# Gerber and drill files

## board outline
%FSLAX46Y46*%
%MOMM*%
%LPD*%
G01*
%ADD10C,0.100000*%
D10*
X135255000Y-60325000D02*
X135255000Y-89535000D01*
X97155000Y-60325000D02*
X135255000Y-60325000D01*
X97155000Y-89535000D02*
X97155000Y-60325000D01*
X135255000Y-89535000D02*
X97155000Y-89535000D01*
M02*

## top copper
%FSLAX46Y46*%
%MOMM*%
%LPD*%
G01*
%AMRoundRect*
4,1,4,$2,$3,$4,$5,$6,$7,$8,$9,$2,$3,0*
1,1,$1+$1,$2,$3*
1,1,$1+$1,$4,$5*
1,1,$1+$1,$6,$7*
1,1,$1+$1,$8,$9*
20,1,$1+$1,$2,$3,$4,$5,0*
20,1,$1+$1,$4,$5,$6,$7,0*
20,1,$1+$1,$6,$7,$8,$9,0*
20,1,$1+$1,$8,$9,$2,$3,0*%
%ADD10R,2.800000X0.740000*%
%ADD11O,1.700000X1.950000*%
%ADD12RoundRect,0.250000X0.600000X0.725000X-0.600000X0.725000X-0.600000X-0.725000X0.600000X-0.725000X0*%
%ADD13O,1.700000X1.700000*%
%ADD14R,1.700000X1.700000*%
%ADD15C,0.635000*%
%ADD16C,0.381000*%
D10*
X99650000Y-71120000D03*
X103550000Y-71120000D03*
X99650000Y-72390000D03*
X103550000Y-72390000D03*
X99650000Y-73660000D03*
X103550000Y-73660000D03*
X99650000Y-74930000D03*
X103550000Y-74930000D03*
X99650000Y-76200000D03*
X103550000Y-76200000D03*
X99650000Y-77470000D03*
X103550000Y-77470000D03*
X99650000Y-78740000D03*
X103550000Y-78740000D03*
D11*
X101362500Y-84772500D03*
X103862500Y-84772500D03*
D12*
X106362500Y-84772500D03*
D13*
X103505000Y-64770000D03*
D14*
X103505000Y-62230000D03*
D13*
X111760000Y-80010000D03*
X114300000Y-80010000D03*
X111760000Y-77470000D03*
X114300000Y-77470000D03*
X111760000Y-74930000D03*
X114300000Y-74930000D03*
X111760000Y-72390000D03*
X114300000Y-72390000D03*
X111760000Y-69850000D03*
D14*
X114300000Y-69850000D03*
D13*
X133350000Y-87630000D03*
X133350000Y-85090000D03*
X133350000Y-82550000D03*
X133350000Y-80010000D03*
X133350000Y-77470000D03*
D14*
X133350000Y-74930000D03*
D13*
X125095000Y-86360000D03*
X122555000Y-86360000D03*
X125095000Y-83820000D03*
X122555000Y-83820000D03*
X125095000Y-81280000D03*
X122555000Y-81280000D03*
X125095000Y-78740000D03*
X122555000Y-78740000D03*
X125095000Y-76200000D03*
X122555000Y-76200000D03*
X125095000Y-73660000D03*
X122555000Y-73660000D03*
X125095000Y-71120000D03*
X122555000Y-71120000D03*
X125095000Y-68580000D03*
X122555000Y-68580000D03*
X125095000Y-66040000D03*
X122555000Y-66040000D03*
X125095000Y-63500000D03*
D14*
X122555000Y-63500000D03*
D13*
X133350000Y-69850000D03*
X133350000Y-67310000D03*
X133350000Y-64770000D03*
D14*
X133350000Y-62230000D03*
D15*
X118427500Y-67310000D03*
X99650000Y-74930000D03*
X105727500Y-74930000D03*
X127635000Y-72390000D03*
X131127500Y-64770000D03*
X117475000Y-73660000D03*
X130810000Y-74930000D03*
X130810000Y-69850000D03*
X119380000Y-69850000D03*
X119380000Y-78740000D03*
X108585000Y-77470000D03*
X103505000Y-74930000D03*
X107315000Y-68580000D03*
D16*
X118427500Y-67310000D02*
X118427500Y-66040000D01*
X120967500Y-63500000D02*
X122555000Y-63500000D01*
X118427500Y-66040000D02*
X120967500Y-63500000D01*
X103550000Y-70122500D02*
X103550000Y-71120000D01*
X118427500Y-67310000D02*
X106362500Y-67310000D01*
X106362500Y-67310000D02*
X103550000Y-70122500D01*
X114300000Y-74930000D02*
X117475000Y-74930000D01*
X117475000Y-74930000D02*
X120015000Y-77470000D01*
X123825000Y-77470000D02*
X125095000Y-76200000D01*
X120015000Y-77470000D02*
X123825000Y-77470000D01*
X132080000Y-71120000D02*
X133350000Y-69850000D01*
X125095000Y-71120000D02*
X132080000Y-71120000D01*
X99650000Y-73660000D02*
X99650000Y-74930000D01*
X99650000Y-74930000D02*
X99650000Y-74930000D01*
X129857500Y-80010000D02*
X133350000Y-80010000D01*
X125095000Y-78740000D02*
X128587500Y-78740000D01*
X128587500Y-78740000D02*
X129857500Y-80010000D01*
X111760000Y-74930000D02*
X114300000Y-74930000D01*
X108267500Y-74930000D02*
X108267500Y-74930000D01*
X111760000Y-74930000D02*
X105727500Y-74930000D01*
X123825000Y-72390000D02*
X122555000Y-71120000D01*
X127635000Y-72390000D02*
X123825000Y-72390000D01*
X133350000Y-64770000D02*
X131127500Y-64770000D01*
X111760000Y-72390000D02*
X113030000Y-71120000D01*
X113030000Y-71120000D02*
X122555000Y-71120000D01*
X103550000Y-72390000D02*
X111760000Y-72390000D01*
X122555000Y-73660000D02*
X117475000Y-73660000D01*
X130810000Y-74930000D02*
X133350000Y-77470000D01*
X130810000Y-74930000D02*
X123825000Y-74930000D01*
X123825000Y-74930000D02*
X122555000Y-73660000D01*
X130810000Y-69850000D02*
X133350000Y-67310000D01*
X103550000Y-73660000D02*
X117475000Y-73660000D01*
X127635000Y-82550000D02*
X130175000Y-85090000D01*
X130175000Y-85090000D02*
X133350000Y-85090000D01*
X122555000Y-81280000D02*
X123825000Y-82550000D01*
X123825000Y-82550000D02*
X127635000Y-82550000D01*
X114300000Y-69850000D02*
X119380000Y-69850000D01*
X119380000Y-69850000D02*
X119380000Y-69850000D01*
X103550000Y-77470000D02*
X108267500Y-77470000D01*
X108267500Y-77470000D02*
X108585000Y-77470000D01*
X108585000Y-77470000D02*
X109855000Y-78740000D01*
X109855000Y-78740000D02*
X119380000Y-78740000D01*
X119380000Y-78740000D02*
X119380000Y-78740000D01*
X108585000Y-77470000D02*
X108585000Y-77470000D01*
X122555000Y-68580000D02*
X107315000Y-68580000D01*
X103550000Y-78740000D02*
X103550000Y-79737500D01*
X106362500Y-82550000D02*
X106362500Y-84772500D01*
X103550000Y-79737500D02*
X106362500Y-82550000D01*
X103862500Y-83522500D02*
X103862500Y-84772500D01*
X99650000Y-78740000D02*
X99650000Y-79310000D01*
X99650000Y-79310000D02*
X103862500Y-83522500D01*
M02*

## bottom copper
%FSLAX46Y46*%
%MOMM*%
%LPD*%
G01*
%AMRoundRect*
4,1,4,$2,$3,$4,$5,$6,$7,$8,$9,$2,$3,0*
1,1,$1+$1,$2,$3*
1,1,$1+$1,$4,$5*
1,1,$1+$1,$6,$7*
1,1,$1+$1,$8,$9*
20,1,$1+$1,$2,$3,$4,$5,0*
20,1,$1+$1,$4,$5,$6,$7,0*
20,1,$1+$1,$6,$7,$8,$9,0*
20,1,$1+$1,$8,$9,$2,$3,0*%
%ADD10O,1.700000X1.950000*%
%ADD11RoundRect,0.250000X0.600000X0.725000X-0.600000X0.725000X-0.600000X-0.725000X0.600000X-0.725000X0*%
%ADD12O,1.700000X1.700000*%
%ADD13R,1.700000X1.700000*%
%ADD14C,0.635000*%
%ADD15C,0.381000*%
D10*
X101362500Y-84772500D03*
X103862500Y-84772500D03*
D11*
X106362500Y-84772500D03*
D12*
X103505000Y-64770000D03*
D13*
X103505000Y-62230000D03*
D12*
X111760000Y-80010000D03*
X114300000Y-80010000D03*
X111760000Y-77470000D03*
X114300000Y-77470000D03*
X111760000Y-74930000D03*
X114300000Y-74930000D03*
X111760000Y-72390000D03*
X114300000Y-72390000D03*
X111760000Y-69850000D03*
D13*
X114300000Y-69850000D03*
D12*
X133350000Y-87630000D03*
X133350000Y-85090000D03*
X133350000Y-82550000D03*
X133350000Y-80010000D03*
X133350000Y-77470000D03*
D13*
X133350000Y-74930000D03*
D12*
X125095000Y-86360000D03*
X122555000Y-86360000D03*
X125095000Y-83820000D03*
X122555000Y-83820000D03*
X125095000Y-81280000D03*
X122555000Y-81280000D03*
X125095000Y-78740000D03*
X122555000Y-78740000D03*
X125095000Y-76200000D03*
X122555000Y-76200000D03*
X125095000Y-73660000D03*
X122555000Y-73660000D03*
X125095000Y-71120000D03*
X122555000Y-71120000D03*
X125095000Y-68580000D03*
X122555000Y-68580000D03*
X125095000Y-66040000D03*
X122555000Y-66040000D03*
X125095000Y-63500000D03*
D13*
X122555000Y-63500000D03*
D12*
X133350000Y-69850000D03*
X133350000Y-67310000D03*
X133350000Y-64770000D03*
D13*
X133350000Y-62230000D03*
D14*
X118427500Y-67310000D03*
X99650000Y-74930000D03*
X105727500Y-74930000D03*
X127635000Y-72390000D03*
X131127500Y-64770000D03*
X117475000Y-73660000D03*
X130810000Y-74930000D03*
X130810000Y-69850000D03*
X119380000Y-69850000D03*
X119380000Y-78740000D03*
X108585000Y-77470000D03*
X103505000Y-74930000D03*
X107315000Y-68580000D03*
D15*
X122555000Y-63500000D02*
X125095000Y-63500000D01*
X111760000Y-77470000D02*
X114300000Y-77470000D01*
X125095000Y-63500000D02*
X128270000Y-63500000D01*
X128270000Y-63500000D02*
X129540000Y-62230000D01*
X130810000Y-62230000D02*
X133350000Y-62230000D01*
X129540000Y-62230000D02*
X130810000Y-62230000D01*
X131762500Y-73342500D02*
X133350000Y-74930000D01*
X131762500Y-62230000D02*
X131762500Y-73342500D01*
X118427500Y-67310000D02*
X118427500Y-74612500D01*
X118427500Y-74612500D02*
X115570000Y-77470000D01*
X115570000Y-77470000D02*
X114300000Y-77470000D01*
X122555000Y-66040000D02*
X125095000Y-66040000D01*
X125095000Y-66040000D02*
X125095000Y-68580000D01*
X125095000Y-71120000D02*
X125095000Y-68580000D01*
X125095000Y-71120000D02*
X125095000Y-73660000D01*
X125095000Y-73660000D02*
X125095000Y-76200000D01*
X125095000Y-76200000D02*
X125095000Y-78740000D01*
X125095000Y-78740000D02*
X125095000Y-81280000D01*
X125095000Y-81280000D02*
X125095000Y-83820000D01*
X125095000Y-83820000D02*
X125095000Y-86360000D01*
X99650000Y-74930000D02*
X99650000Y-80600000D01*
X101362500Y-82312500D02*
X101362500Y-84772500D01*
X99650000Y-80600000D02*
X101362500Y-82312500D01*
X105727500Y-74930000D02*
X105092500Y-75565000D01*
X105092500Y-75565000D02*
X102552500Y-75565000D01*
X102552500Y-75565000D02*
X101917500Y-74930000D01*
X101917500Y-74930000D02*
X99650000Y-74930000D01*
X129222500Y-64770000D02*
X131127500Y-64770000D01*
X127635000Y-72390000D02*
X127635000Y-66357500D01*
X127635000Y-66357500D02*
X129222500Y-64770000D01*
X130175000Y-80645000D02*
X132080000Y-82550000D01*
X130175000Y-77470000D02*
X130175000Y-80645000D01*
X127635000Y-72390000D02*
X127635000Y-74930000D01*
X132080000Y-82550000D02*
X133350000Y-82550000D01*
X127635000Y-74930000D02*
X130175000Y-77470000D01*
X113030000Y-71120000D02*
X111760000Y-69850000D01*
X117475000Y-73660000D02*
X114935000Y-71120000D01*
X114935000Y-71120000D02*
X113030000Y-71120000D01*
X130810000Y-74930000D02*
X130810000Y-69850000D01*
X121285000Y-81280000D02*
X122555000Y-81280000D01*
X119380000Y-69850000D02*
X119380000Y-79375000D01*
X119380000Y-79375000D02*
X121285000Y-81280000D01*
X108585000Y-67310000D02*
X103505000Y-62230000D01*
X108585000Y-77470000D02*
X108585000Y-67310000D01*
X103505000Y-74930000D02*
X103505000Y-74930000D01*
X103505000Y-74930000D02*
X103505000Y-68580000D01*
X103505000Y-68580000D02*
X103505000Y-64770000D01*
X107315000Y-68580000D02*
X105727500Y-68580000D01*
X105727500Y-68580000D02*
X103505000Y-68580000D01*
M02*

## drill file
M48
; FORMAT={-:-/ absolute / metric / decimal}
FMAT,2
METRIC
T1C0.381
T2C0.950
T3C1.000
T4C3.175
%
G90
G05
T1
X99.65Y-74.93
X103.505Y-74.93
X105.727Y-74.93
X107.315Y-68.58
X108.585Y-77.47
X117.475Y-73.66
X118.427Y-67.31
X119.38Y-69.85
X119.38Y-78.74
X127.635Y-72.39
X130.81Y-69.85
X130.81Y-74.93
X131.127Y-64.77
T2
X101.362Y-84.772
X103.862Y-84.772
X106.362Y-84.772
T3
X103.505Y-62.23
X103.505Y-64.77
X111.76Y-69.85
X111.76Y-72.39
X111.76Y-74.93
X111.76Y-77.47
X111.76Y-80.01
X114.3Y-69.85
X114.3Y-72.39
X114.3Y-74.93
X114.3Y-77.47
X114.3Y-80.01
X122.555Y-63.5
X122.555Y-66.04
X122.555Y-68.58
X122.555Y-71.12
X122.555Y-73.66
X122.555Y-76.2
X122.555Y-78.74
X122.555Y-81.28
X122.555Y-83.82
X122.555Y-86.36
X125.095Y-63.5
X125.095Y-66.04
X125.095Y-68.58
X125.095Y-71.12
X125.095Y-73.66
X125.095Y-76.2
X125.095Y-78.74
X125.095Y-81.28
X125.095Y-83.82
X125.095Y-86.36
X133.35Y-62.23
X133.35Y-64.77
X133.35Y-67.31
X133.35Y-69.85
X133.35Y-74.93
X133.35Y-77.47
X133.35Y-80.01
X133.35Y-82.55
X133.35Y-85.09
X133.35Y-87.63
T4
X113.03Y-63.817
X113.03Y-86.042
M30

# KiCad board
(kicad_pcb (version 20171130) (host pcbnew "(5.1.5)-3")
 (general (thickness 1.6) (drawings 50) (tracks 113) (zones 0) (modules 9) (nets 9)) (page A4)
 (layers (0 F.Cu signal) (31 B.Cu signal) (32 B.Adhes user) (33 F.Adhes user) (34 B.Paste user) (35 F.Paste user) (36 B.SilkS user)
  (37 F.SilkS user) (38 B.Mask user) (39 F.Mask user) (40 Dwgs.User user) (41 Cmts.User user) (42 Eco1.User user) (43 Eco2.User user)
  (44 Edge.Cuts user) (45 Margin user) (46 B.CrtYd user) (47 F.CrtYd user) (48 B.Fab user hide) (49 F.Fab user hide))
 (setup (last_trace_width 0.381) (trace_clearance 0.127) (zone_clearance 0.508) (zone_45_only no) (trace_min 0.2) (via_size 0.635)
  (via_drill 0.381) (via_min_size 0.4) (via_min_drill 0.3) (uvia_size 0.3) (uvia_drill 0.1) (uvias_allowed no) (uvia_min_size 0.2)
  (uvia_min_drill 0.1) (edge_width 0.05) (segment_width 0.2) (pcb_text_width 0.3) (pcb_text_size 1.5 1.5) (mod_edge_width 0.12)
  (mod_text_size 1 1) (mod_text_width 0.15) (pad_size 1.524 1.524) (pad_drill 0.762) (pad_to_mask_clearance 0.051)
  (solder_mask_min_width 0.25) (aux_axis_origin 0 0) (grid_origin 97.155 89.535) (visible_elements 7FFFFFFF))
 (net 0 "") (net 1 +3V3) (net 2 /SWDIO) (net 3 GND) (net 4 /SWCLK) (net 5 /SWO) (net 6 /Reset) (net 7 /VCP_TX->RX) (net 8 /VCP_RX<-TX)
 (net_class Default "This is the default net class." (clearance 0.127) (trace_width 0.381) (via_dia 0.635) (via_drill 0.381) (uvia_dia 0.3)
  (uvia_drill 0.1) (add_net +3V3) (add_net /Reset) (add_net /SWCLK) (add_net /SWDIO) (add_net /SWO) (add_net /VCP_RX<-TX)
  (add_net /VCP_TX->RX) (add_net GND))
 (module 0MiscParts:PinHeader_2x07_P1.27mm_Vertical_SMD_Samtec (layer F.Cu) (at 101.6 74.93)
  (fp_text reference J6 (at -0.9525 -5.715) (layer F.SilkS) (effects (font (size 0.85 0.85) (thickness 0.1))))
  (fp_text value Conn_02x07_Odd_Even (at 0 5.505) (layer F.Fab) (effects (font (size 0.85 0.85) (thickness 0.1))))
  (pad 1 smd rect (at -1.95 -3.81) (size 2.8 0.74) (layers F.Cu F.Paste F.Mask))
  (pad 2 smd rect (at 1.95 -3.81) (size 2.8 0.74) (layers F.Cu F.Paste F.Mask) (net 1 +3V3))
  (pad 3 smd rect (at -1.95 -2.54) (size 2.8 0.74) (layers F.Cu F.Paste F.Mask))
  (pad 4 smd rect (at 1.95 -2.54) (size 2.8 0.74) (layers F.Cu F.Paste F.Mask) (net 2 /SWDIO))
  (pad 5 smd rect (at -1.95 -1.27) (size 2.8 0.74) (layers F.Cu F.Paste F.Mask) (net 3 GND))
  (pad 6 smd rect (at 1.95 -1.27) (size 2.8 0.74) (layers F.Cu F.Paste F.Mask) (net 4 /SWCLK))
  (pad 7 smd rect (at -1.95 0) (size 2.8 0.74) (layers F.Cu F.Paste F.Mask) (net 3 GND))
  (pad 8 smd rect (at 1.95 0) (size 2.8 0.74) (layers F.Cu F.Paste F.Mask) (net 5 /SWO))
  (pad 9 smd rect (at -1.95 1.27) (size 2.8 0.74) (layers F.Cu F.Paste F.Mask))
  (pad 10 smd rect (at 1.95 1.27) (size 2.8 0.74) (layers F.Cu F.Paste F.Mask))
  (pad 11 smd rect (at -1.95 2.54) (size 2.8 0.74) (layers F.Cu F.Paste F.Mask))
  (pad 12 smd rect (at 1.95 2.54) (size 2.8 0.74) (layers F.Cu F.Paste F.Mask) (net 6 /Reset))
  (pad 13 smd rect (at -1.95 3.81) (size 2.8 0.74) (layers F.Cu F.Paste F.Mask) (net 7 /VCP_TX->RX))
  (pad 14 smd rect (at 1.95 3.81) (size 2.8 0.74) (layers F.Cu F.Paste F.Mask) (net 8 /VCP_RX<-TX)))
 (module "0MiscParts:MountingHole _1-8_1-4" (layer F.Cu) (at 113.03 63.8175)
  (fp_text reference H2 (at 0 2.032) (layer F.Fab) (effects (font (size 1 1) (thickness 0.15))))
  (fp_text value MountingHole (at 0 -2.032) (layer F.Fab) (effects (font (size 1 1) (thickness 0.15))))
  (pad "" np_thru_hole circle (at 0 0) (size 3.175 3.175) (drill 3.175) (layers *.Cu *.Mask)))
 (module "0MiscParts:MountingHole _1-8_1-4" (layer F.Cu) (at 113.03 86.0425)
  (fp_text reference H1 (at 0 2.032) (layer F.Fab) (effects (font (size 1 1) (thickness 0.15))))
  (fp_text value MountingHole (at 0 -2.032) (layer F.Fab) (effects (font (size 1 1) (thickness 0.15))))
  (pad "" np_thru_hole circle (at 0 0) (size 3.175 3.175) (drill 3.175) (layers *.Cu *.Mask)))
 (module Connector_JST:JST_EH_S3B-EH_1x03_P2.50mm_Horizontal (layer F.Cu) (at 106.3625 84.7725 180)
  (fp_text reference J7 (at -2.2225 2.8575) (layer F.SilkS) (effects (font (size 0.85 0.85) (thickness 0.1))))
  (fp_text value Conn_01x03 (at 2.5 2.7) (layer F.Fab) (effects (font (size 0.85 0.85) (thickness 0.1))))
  (pad 3 thru_hole oval (at 5 0 180) (size 1.7 1.95) (drill 0.95) (layers *.Cu *.Mask) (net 3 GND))
  (pad 2 thru_hole oval (at 2.5 0 180) (size 1.7 1.95) (drill 0.95) (layers *.Cu *.Mask) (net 7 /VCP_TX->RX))
  (pad 1 thru_hole roundrect (at 0 0 180) (size 1.7 1.95) (drill 0.95) (layers *.Cu *.Mask) (roundrect_rratio 0.147059) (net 8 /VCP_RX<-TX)))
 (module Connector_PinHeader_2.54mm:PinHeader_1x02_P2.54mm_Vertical (layer F.Cu) (at 103.505 62.23)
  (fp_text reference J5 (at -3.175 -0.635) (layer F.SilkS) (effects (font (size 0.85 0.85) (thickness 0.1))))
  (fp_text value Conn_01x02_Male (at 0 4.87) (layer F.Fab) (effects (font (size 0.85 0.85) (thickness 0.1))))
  (pad 2 thru_hole oval (at 0 2.54) (size 1.7 1.7) (drill 1) (layers *.Cu *.Mask) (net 5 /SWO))
  (pad 1 thru_hole rect (at 0 0) (size 1.7 1.7) (drill 1) (layers *.Cu *.Mask) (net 6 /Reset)))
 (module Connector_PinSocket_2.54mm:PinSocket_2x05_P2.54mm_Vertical (layer F.Cu) (at 114.3 69.85)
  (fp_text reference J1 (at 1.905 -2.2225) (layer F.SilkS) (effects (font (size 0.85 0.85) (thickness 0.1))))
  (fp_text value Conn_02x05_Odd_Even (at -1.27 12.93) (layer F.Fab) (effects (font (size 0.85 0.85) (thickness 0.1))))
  (pad 10 thru_hole oval (at -2.54 10.16) (size 1.7 1.7) (drill 1) (layers *.Cu *.Mask))
  (pad 9 thru_hole oval (at 0 10.16) (size 1.7 1.7) (drill 1) (layers *.Cu *.Mask))
  (pad 8 thru_hole oval (at -2.54 7.62) (size 1.7 1.7) (drill 1) (layers *.Cu *.Mask) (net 1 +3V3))
  (pad 7 thru_hole oval (at 0 7.62) (size 1.7 1.7) (drill 1) (layers *.Cu *.Mask) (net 1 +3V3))
  (pad 6 thru_hole oval (at -2.54 5.08) (size 1.7 1.7) (drill 1) (layers *.Cu *.Mask) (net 3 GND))
  (pad 5 thru_hole oval (at 0 5.08) (size 1.7 1.7) (drill 1) (layers *.Cu *.Mask) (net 3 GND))
  (pad 4 thru_hole oval (at -2.54 2.54) (size 1.7 1.7) (drill 1) (layers *.Cu *.Mask) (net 2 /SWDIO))
  (pad 3 thru_hole oval (at 0 2.54) (size 1.7 1.7) (drill 1) (layers *.Cu *.Mask))
  (pad 2 thru_hole oval (at -2.54 0) (size 1.7 1.7) (drill 1) (layers *.Cu *.Mask) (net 4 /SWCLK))
  (pad 1 thru_hole rect (at 0 0) (size 1.7 1.7) (drill 1) (layers *.Cu *.Mask) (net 6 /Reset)))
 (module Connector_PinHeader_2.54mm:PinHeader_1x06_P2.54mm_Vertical (layer F.Cu) (at 133.35 74.93)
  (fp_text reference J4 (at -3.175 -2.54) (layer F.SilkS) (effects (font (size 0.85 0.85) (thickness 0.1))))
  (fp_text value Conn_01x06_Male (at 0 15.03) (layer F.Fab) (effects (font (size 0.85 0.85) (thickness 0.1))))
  (pad 6 thru_hole oval (at 0 12.7) (size 1.7 1.7) (drill 1) (layers *.Cu *.Mask))
  (pad 5 thru_hole oval (at 0 10.16) (size 1.7 1.7) (drill 1) (layers *.Cu *.Mask) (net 6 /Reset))
  (pad 4 thru_hole oval (at 0 7.62) (size 1.7 1.7) (drill 1) (layers *.Cu *.Mask) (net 2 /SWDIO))
  (pad 3 thru_hole oval (at 0 5.08) (size 1.7 1.7) (drill 1) (layers *.Cu *.Mask) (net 3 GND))
  (pad 2 thru_hole oval (at 0 2.54) (size 1.7 1.7) (drill 1) (layers *.Cu *.Mask) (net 4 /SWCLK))
  (pad 1 thru_hole rect (at 0 0) (size 1.7 1.7) (drill 1) (layers *.Cu *.Mask) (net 1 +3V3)))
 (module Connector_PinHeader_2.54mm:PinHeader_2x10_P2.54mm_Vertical (layer F.Cu) (at 122.555 63.5)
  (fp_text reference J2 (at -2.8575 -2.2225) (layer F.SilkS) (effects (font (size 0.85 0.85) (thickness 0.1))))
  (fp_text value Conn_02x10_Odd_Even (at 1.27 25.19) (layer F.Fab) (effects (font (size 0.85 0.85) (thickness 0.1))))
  (pad 20 thru_hole oval (at 2.54 22.86) (size 1.7 1.7) (drill 1) (layers *.Cu *.Mask) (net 3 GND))
  (pad 19 thru_hole oval (at 0 22.86) (size 1.7 1.7) (drill 1) (layers *.Cu *.Mask))
  (pad 18 thru_hole oval (at 2.54 20.32) (size 1.7 1.7) (drill 1) (layers *.Cu *.Mask) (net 3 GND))
  (pad 17 thru_hole oval (at 0 20.32) (size 1.7 1.7) (drill 1) (layers *.Cu *.Mask))
  (pad 16 thru_hole oval (at 2.54 17.78) (size 1.7 1.7) (drill 1) (layers *.Cu *.Mask) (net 3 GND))
  (pad 15 thru_hole oval (at 0 17.78) (size 1.7 1.7) (drill 1) (layers *.Cu *.Mask) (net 6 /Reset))
  (pad 14 thru_hole oval (at 2.54 15.24) (size 1.7 1.7) (drill 1) (layers *.Cu *.Mask) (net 3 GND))
  (pad 13 thru_hole oval (at 0 15.24) (size 1.7 1.7) (drill 1) (layers *.Cu *.Mask))
  (pad 12 thru_hole oval (at 2.54 12.7) (size 1.7 1.7) (drill 1) (layers *.Cu *.Mask) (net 3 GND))
  (pad 11 thru_hole oval (at 0 12.7) (size 1.7 1.7) (drill 1) (layers *.Cu *.Mask))
  (pad 10 thru_hole oval (at 2.54 10.16) (size 1.7 1.7) (drill 1) (layers *.Cu *.Mask) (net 3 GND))
  (pad 9 thru_hole oval (at 0 10.16) (size 1.7 1.7) (drill 1) (layers *.Cu *.Mask) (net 4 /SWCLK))
  (pad 8 thru_hole oval (at 2.54 7.62) (size 1.7 1.7) (drill 1) (layers *.Cu *.Mask) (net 3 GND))
  (pad 7 thru_hole oval (at 0 7.62) (size 1.7 1.7) (drill 1) (layers *.Cu *.Mask) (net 2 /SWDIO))
  (pad 6 thru_hole oval (at 2.54 5.08) (size 1.7 1.7) (drill 1) (layers *.Cu *.Mask) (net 3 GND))
  (pad 5 thru_hole oval (at 0 5.08) (size 1.7 1.7) (drill 1) (layers *.Cu *.Mask) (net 5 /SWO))
  (pad 4 thru_hole oval (at 2.54 2.54) (size 1.7 1.7) (drill 1) (layers *.Cu *.Mask) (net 3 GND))
  (pad 3 thru_hole oval (at 0 2.54) (size 1.7 1.7) (drill 1) (layers *.Cu *.Mask) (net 3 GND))
  (pad 2 thru_hole oval (at 2.54 0) (size 1.7 1.7) (drill 1) (layers *.Cu *.Mask) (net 1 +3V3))
  (pad 1 thru_hole rect (at 0 0) (size 1.7 1.7) (drill 1) (layers *.Cu *.Mask) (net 1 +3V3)))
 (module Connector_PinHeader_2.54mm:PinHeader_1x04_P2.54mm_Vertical (layer F.Cu) (at 133.35 62.23)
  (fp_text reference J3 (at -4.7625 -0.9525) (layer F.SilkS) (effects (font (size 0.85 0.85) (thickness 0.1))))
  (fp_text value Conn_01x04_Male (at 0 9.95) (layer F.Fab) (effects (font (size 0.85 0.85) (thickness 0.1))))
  (pad 4 thru_hole oval (at 0 7.62) (size 1.7 1.7) (drill 1) (layers *.Cu *.Mask) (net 3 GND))
  (pad 3 thru_hole oval (at 0 5.08) (size 1.7 1.7) (drill 1) (layers *.Cu *.Mask) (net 4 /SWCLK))
  (pad 2 thru_hole oval (at 0 2.54) (size 1.7 1.7) (drill 1) (layers *.Cu *.Mask) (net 2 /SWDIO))
  (pad 1 thru_hole rect (at 0 0) (size 1.7 1.7) (drill 1) (layers *.Cu *.Mask) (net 1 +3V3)))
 (gr_line (start 135.255 60.325) (end 135.255 89.535) (layer Edge.Cuts) (width 0.1))
 (gr_line (start 97.155 60.325) (end 135.255 60.325) (layer Edge.Cuts) (width 0.1))
 (gr_line (start 97.155 89.535) (end 97.155 60.325) (layer Edge.Cuts) (width 0.1))
 (gr_line (start 135.255 89.535) (end 97.155 89.535) (layer Edge.Cuts) (width 0.1))
 (segment (start 122.555 63.5) (end 125.095 63.5) (width 0.381) (layer B.Cu) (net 1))
 (segment (start 111.76 77.47) (end 114.3 77.47) (width 0.381) (layer B.Cu) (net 1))
 (segment (start 125.095 63.5) (end 128.27 63.5) (width 0.381) (layer B.Cu) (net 1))
 (segment (start 128.27 63.5) (end 129.54 62.23) (width 0.381) (layer B.Cu) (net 1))
 (segment (start 130.81 62.23) (end 133.35 62.23) (width 0.381) (layer B.Cu) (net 1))
 (segment (start 129.54 62.23) (end 130.81 62.23) (width 0.381) (layer B.Cu) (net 1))
 (segment (start 131.7625 73.3425) (end 133.35 74.93) (width 0.381) (layer B.Cu) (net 1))
 (segment (start 131.7625 62.23) (end 131.7625 73.3425) (width 0.381) (layer B.Cu) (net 1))
 (segment (start 118.4275 67.31) (end 118.4275 74.6125) (width 0.381) (layer B.Cu) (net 1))
 (segment (start 118.4275 74.6125) (end 115.57 77.47) (width 0.381) (layer B.Cu) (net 1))
 (via (at 118.4275 67.31) (size 0.635) (drill 0.381) (layers F.Cu B.Cu) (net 1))
 (segment (start 115.57 77.47) (end 114.3 77.47) (width 0.381) (layer B.Cu) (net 1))
 (segment (start 118.4275 67.31) (end 118.4275 66.04) (width 0.381) (layer F.Cu) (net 1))
 (segment (start 120.9675 63.5) (end 122.555 63.5) (width 0.381) (layer F.Cu) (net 1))
 (segment (start 118.4275 66.04) (end 120.9675 63.5) (width 0.381) (layer F.Cu) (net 1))
 (segment (start 103.55 70.1225) (end 103.55 71.12) (width 0.381) (layer F.Cu) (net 1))
 (segment (start 118.4275 67.31) (end 106.3625 67.31) (width 0.381) (layer F.Cu) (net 1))
 (segment (start 106.3625 67.31) (end 103.55 70.1225) (width 0.381) (layer F.Cu) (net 1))
 (segment (start 122.555 66.04) (end 125.095 66.04) (width 0.381) (layer B.Cu) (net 3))
 (segment (start 125.095 66.04) (end 125.095 68.58) (width 0.381) (layer B.Cu) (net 3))
 (segment (start 125.095 71.12) (end 125.095 68.58) (width 0.381) (layer B.Cu) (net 3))
 (segment (start 125.095 71.12) (end 125.095 73.66) (width 0.381) (layer B.Cu) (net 3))
 (segment (start 125.095 73.66) (end 125.095 76.2) (width 0.381) (layer B.Cu) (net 3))
 (segment (start 125.095 76.2) (end 125.095 78.74) (width 0.381) (layer B.Cu) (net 3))
 (segment (start 125.095 78.74) (end 125.095 81.28) (width 0.381) (layer B.Cu) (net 3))
 (segment (start 125.095 81.28) (end 125.095 83.82) (width 0.381) (layer B.Cu) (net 3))
 (segment (start 125.095 83.82) (end 125.095 86.36) (width 0.381) (layer B.Cu) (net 3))
 (segment (start 114.3 74.93) (end 117.475 74.93) (width 0.381) (layer F.Cu) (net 3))
 (segment (start 117.475 74.93) (end 120.015 77.47) (width 0.381) (layer F.Cu) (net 3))
 (segment (start 123.825 77.47) (end 125.095 76.2) (width 0.381) (layer F.Cu) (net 3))
 (segment (start 120.015 77.47) (end 123.825 77.47) (width 0.381) (layer F.Cu) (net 3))
 (segment (start 132.08 71.12) (end 133.35 69.85) (width 0.381) (layer F.Cu) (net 3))
 (segment (start 125.095 71.12) (end 132.08 71.12) (width 0.381) (layer F.Cu) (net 3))
 (segment (start 99.65 73.66) (end 99.65 74.93) (width 0.381) (layer F.Cu) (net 3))
 (segment (start 99.65 74.93) (end 99.65 74.93) (width 0.381) (layer F.Cu) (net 3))
 (via (at 99.65 74.93) (size 0.635) (drill 0.381) (layers F.Cu B.Cu) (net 3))
 (segment (start 99.65 74.93) (end 99.65 80.6) (width 0.381) (layer B.Cu) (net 3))
 (segment (start 101.3625 82.3125) (end 101.3625 84.7725) (width 0.381) (layer B.Cu) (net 3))
 (segment (start 99.65 80.6) (end 101.3625 82.3125) (width 0.381) (layer B.Cu) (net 3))
 (segment (start 129.8575 80.01) (end 133.35 80.01) (width 0.381) (layer F.Cu) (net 3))
 (segment (start 125.095 78.74) (end 128.5875 78.74) (width 0.381) (layer F.Cu) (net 3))
 (segment (start 128.5875 78.74) (end 129.8575 80.01) (width 0.381) (layer F.Cu) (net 3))
 (segment (start 111.76 74.93) (end 114.3 74.93) (width 0.381) (layer F.Cu) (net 3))
 (segment (start 108.2675 74.93) (end 108.2675 74.93) (width 0.381) (layer F.Cu) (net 3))
 (segment (start 111.76 74.93) (end 105.7275 74.93) (width 0.381) (layer F.Cu) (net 3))
 (segment (start 105.7275 74.93) (end 105.0925 75.565) (width 0.381) (layer B.Cu) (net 3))
 (segment (start 105.0925 75.565) (end 102.5525 75.565) (width 0.381) (layer B.Cu) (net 3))
 (via (at 105.7275 74.93) (size 0.635) (drill 0.381) (layers F.Cu B.Cu) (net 3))
 (segment (start 102.5525 75.565) (end 101.9175 74.93) (width 0.381) (layer B.Cu) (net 3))
 (segment (start 101.9175 74.93) (end 99.65 74.93) (width 0.381) (layer B.Cu) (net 3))
 (via (at 127.635 72.39) (size 0.635) (drill 0.381) (layers F.Cu B.Cu) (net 2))
 (segment (start 123.825 72.39) (end 122.555 71.12) (width 0.381) (layer F.Cu) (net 2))
 (segment (start 127.635 72.39) (end 123.825 72.39) (width 0.381) (layer F.Cu) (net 2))
 (segment (start 133.35 64.77) (end 131.1275 64.77) (width 0.381) (layer F.Cu) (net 2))
 (via (at 131.1275 64.77) (size 0.635) (drill 0.381) (layers F.Cu B.Cu) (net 2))
 (segment (start 129.2225 64.77) (end 131.1275 64.77) (width 0.381) (layer B.Cu) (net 2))
 (segment (start 127.635 72.39) (end 127.635 66.3575) (width 0.381) (layer B.Cu) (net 2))
 (segment (start 127.635 66.3575) (end 129.2225 64.77) (width 0.381) (layer B.Cu) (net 2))
 (segment (start 130.175 80.645) (end 132.08 82.55) (width 0.381) (layer B.Cu) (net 2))
 (segment (start 130.175 77.47) (end 130.175 80.645) (width 0.381) (layer B.Cu) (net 2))
 (segment (start 127.635 72.39) (end 127.635 74.93) (width 0.381) (layer B.Cu) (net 2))
 (segment (start 132.08 82.55) (end 133.35 82.55) (width 0.381) (layer B.Cu) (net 2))
 (segment (start 127.635 74.93) (end 130.175 77.47) (width 0.381) (layer B.Cu) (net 2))
 (segment (start 111.76 72.39) (end 113.03 71.12) (width 0.381) (layer F.Cu) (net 2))
 (segment (start 113.03 71.12) (end 122.555 71.12) (width 0.381) (layer F.Cu) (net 2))
 (segment (start 103.55 72.39) (end 111.76 72.39) (width 0.381) (layer F.Cu) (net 2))
 (via (at 117.475 73.66) (size 0.635) (drill 0.381) (layers F.Cu B.Cu) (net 4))
 (segment (start 122.555 73.66) (end 117.475 73.66) (width 0.381) (layer F.Cu) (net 4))
 (segment (start 113.03 71.12) (end 111.76 69.85) (width 0.381) (layer B.Cu) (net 4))
 (segment (start 117.475 73.66) (end 114.935 71.12) (width 0.381) (layer B.Cu) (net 4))
 (segment (start 114.935 71.12) (end 113.03 71.12) (width 0.381) (layer B.Cu) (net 4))
 (segment (start 130.81 74.93) (end 133.35 77.47) (width 0.381) (layer F.Cu) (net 4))
 (via (at 130.81 74.93) (size 0.635) (drill 0.381) (layers F.Cu B.Cu) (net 4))
 (segment (start 130.81 74.93) (end 123.825 74.93) (width 0.381) (layer F.Cu) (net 4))
 (segment (start 123.825 74.93) (end 122.555 73.66) (width 0.381) (layer F.Cu) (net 4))
 (segment (start 130.81 69.85) (end 133.35 67.31) (width 0.381) (layer F.Cu) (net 4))
 (via (at 130.81 69.85) (size 0.635) (drill 0.381) (layers F.Cu B.Cu) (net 4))
 (segment (start 130.81 74.93) (end 130.81 69.85) (width 0.381) (layer B.Cu) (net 4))
 (segment (start 103.55 73.66) (end 117.475 73.66) (width 0.381) (layer F.Cu) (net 4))
 (segment (start 127.635 82.55) (end 130.175 85.09) (width 0.381) (layer F.Cu) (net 6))
 (segment (start 130.175 85.09) (end 133.35 85.09) (width 0.381) (layer F.Cu) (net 6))
 (segment (start 122.555 81.28) (end 123.825 82.55) (width 0.381) (layer F.Cu) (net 6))
 (segment (start 123.825 82.55) (end 127.635 82.55) (width 0.381) (layer F.Cu) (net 6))
 (segment (start 114.3 69.85) (end 119.38 69.85) (width 0.381) (layer F.Cu) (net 6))
 (segment (start 119.38 69.85) (end 119.38 69.85) (width 0.381) (layer F.Cu) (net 6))
 (via (at 119.38 69.85) (size 0.635) (drill 0.381) (layers F.Cu B.Cu) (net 6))
 (segment (start 103.55 77.47) (end 108.2675 77.47) (width 0.381) (layer F.Cu) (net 6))
 (segment (start 108.2675 77.47) (end 108.585 77.47) (width 0.381) (layer F.Cu) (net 6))
 (segment (start 108.585 77.47) (end 109.855 78.74) (width 0.381) (layer F.Cu) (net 6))
 (segment (start 109.855 78.74) (end 119.38 78.74) (width 0.381) (layer F.Cu) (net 6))
 (segment (start 121.285 81.28) (end 122.555 81.28) (width 0.381) (layer B.Cu) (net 6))
 (segment (start 119.38 69.85) (end 119.38 79.375) (width 0.381) (layer B.Cu) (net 6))
 (segment (start 119.38 79.375) (end 121.285 81.28) (width 0.381) (layer B.Cu) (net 6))
 (segment (start 119.38 78.74) (end 119.38 78.74) (width 0.381) (layer F.Cu) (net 6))
 (via (at 119.38 78.74) (size 0.635) (drill 0.381) (layers F.Cu B.Cu) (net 6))
 (segment (start 108.585 77.47) (end 108.585 77.47) (width 0.381) (layer F.Cu) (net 6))
 (via (at 108.585 77.47) (size 0.635) (drill 0.381) (layers F.Cu B.Cu) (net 6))
 (segment (start 108.585 67.31) (end 103.505 62.23) (width 0.381) (layer B.Cu) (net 6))
 (segment (start 108.585 77.47) (end 108.585 67.31) (width 0.381) (layer B.Cu) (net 6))
 (segment (start 103.505 74.93) (end 103.505 74.93) (width 0.381) (layer B.Cu) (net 5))
 (via (at 103.505 74.93) (size 0.635) (drill 0.381) (layers F.Cu B.Cu) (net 5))
 (segment (start 103.505 74.93) (end 103.505 68.58) (width 0.381) (layer B.Cu) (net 5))
 (segment (start 103.505 68.58) (end 103.505 64.77) (width 0.381) (layer B.Cu) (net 5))
 (segment (start 107.315 68.58) (end 105.7275 68.58) (width 0.381) (layer B.Cu) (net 5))
 (via (at 107.315 68.58) (size 0.635) (drill 0.381) (layers F.Cu B.Cu) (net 5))
 (segment (start 105.7275 68.58) (end 103.505 68.58) (width 0.381) (layer B.Cu) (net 5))
 (segment (start 122.555 68.58) (end 107.315 68.58) (width 0.381) (layer F.Cu) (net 5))
 (segment (start 103.55 78.74) (end 103.55 79.7375) (width 0.381) (layer F.Cu) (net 8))
 (segment (start 106.3625 82.55) (end 106.3625 84.7725) (width 0.381) (layer F.Cu) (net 8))
 (segment (start 103.55 79.7375) (end 106.3625 82.55) (width 0.381) (layer F.Cu) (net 8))
 (segment (start 103.8625 83.5225) (end 103.8625 84.7725) (width 0.381) (layer F.Cu) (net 7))
 (segment (start 99.65 78.74) (end 99.65 79.31) (width 0.381) (layer F.Cu) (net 7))
 (segment (start 99.65 79.31) (end 103.8625 83.5225) (width 0.381) (layer F.Cu) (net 7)))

